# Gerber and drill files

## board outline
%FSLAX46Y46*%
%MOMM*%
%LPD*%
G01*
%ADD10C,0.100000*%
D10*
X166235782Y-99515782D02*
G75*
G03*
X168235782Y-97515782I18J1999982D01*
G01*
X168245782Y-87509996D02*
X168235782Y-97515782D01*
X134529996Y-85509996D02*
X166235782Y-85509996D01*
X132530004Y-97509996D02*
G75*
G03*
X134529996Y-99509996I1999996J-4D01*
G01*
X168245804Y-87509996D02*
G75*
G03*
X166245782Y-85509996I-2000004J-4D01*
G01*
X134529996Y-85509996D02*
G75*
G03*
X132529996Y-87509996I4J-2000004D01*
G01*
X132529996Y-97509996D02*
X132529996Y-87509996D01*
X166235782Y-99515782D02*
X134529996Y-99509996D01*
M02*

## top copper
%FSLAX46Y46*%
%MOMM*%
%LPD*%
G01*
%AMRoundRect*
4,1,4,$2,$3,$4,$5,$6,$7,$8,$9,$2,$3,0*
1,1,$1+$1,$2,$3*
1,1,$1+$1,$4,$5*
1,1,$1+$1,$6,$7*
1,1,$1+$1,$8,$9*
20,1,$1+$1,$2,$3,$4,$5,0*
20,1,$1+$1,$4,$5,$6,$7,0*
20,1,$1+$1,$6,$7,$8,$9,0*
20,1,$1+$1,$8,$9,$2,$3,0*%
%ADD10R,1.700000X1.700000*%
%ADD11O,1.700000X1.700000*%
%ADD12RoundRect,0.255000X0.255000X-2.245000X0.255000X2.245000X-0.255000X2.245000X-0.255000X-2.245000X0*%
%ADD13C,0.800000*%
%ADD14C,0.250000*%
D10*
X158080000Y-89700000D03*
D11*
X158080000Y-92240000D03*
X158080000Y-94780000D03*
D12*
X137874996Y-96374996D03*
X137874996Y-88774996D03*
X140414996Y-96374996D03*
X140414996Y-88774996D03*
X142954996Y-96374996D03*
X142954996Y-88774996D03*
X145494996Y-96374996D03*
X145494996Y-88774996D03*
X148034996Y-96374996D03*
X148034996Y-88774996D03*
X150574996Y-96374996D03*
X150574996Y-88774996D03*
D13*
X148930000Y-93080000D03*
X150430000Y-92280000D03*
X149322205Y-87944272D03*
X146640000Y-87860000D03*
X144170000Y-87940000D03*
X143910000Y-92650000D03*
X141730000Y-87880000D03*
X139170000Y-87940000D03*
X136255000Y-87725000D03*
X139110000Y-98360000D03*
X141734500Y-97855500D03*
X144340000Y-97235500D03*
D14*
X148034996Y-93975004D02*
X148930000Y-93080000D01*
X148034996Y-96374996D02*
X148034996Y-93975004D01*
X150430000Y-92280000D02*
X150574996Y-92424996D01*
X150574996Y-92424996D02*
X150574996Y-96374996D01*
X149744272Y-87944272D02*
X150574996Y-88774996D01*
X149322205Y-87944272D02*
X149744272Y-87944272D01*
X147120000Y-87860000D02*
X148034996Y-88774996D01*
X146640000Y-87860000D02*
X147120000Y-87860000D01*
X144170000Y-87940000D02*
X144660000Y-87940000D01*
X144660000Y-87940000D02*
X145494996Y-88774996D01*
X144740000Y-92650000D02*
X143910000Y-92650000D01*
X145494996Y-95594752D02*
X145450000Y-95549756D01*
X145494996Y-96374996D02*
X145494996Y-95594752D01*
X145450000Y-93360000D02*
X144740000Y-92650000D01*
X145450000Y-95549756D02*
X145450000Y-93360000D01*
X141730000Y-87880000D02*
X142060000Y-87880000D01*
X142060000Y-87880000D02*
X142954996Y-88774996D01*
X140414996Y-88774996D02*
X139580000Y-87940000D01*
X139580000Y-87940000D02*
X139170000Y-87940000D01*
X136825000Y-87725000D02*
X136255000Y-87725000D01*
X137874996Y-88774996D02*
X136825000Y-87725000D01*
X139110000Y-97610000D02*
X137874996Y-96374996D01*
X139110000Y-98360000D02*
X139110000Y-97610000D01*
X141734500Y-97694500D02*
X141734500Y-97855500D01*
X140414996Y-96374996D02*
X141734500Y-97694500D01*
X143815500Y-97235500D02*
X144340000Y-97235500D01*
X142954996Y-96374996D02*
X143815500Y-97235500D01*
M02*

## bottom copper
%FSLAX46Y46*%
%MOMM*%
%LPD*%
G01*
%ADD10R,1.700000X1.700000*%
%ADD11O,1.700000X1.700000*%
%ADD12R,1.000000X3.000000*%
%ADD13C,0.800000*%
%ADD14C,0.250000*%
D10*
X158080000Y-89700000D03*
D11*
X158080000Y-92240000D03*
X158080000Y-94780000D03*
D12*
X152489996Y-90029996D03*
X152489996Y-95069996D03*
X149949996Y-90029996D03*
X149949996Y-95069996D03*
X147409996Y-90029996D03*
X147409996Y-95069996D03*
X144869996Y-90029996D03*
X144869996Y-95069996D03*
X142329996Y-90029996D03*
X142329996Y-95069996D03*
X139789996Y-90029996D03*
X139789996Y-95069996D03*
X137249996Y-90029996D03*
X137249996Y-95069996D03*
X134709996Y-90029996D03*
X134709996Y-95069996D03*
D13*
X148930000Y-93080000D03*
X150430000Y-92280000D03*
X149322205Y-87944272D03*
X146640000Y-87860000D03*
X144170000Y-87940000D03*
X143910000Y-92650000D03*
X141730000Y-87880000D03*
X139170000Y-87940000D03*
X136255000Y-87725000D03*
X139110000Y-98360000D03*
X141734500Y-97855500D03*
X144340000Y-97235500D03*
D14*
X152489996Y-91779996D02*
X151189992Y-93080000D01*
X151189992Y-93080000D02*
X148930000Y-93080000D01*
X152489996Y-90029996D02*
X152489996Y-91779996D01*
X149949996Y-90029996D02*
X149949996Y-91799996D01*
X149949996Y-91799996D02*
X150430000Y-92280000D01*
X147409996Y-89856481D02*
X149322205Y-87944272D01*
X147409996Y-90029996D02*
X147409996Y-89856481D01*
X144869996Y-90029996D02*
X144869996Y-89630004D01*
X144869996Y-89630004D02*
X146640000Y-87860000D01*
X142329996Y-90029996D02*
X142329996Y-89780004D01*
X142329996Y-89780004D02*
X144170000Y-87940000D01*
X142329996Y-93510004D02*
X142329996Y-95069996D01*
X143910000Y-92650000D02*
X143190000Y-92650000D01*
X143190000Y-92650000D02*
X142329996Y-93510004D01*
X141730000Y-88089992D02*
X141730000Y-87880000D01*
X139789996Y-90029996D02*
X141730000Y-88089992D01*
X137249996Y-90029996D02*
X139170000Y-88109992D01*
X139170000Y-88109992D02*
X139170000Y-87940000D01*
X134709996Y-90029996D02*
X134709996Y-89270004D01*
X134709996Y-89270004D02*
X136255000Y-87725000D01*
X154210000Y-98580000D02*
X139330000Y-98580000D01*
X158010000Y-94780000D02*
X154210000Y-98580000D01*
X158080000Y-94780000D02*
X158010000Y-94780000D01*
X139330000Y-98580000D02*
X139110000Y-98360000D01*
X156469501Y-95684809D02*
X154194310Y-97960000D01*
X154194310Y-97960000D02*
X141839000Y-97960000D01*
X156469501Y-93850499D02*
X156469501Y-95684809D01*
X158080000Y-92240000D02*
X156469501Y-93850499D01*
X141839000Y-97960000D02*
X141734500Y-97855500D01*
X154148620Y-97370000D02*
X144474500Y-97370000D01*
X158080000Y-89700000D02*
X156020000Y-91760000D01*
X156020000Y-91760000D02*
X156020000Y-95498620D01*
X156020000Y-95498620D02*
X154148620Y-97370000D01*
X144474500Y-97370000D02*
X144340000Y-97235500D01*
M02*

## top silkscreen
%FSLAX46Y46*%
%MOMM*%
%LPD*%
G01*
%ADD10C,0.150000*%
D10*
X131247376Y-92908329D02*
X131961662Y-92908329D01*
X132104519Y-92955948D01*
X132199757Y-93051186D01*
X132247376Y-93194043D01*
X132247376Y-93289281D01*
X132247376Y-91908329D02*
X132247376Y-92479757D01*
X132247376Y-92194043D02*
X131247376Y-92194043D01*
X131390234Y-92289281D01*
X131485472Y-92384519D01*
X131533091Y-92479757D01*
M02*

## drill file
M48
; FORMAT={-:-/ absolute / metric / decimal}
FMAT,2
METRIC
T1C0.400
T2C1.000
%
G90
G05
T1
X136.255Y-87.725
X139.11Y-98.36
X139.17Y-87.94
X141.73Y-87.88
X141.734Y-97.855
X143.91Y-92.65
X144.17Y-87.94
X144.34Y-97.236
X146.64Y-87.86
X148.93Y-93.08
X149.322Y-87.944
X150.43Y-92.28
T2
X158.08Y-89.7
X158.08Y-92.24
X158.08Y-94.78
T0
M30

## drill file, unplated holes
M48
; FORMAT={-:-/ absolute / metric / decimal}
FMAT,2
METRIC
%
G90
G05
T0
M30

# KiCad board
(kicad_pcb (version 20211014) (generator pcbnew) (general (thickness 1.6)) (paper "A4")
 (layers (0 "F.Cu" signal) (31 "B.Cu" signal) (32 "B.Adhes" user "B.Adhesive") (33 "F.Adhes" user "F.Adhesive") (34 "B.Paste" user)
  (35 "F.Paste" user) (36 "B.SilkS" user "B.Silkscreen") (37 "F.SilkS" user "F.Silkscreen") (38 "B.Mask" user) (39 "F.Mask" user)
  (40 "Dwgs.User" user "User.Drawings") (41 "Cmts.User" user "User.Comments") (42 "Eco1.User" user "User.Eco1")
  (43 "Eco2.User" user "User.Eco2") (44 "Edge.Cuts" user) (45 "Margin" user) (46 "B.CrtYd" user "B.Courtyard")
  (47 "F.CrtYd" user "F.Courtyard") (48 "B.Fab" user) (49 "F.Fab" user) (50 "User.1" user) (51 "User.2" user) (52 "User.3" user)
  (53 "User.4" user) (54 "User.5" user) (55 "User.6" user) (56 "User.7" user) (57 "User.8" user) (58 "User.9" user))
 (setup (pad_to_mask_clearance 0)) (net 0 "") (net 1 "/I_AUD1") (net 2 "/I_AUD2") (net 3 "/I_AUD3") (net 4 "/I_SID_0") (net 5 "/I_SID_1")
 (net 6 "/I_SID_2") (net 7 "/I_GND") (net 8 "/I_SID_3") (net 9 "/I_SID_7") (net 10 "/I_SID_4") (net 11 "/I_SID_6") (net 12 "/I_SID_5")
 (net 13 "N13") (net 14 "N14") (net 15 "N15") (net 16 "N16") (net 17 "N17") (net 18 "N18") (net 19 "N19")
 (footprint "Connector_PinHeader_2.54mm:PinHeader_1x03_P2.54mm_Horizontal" (layer "F.Cu") (at 158.08 89.7)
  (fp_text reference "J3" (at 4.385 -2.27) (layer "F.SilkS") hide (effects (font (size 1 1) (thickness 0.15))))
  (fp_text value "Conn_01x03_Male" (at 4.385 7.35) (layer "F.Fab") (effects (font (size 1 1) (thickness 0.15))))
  (pad "1" thru_hole rect (at 0 0) (size 1.7 1.7) (drill 1) (layers *.Cu *.Mask) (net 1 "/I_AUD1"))
  (pad "2" thru_hole oval (at 0 2.54) (size 1.7 1.7) (drill 1) (layers *.Cu *.Mask) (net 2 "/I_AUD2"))
  (pad "3" thru_hole oval (at 0 5.08) (size 1.7 1.7) (drill 1) (layers *.Cu *.Mask) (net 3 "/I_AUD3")))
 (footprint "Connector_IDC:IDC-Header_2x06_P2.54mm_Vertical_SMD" (layer "F.Cu") (at 144.224996 92.574996 90)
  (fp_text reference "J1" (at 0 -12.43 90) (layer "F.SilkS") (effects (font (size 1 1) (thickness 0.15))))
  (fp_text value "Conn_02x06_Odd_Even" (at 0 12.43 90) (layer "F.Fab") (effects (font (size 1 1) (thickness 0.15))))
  (pad "1" smd roundrect (at -3.8 -6.35 90) (size 5 1.02) (layers "F.Cu" "F.Paste" "F.Mask") (roundrect_rratio 0.25) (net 3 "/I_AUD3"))
  (pad "2" smd roundrect (at 3.8 -6.35 90) (size 5 1.02) (layers "F.Cu" "F.Paste" "F.Mask") (roundrect_rratio 0.25) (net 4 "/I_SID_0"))
  (pad "3" smd roundrect (at -3.8 -3.81 90) (size 5 1.02) (layers "F.Cu" "F.Paste" "F.Mask") (roundrect_rratio 0.25) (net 2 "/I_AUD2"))
  (pad "4" smd roundrect (at 3.8 -3.81 90) (size 5 1.02) (layers "F.Cu" "F.Paste" "F.Mask") (roundrect_rratio 0.25) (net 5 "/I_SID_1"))
  (pad "5" smd roundrect (at -3.8 -1.27 90) (size 5 1.02) (layers "F.Cu" "F.Paste" "F.Mask") (roundrect_rratio 0.25) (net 1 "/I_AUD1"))
  (pad "6" smd roundrect (at 3.8 -1.27 90) (size 5 1.02) (layers "F.Cu" "F.Paste" "F.Mask") (roundrect_rratio 0.25) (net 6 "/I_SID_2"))
  (pad "7" smd roundrect (at -3.8 1.27 90) (size 5 1.02) (layers "F.Cu" "F.Paste" "F.Mask") (roundrect_rratio 0.25) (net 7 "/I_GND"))
  (pad "8" smd roundrect (at 3.8 1.27 90) (size 5 1.02) (layers "F.Cu" "F.Paste" "F.Mask") (roundrect_rratio 0.25) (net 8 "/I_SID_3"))
  (pad "9" smd roundrect (at -3.8 3.81 90) (size 5 1.02) (layers "F.Cu" "F.Paste" "F.Mask") (roundrect_rratio 0.25) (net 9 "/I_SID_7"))
  (pad "10" smd roundrect (at 3.8 3.81 90) (size 5 1.02) (layers "F.Cu" "F.Paste" "F.Mask") (roundrect_rratio 0.25) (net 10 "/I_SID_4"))
  (pad "11" smd roundrect (at -3.8 6.35 90) (size 5 1.02) (layers "F.Cu" "F.Paste" "F.Mask") (roundrect_rratio 0.25) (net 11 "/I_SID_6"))
  (pad "12" smd roundrect (at 3.8 6.35 90) (size 5 1.02) (layers "F.Cu" "F.Paste" "F.Mask") (roundrect_rratio 0.25) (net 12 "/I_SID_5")))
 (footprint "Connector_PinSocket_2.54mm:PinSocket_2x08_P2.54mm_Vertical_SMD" (layer "B.Cu") (at 143.599996 92.549996 90)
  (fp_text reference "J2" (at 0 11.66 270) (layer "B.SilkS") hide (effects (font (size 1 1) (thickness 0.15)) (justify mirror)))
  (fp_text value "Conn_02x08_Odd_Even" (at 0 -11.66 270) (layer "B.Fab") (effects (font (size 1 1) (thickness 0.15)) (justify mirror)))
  (pad "1" smd rect (at 2.52 8.89 90) (size 3 1) (layers "B.Cu" "B.Paste" "B.Mask") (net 9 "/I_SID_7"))
  (pad "2" smd rect (at -2.52 8.89 90) (size 3 1) (layers "B.Cu" "B.Paste" "B.Mask") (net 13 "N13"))
  (pad "3" smd rect (at 2.52 6.35 90) (size 3 1) (layers "B.Cu" "B.Paste" "B.Mask") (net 11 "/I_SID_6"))
  (pad "4" smd rect (at -2.52 6.35 90) (size 3 1) (layers "B.Cu" "B.Paste" "B.Mask") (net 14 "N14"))
  (pad "5" smd rect (at 2.52 3.81 90) (size 3 1) (layers "B.Cu" "B.Paste" "B.Mask") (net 12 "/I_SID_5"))
  (pad "6" smd rect (at -2.52 3.81 90) (size 3 1) (layers "B.Cu" "B.Paste" "B.Mask") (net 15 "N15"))
  (pad "7" smd rect (at 2.52 1.27 90) (size 3 1) (layers "B.Cu" "B.Paste" "B.Mask") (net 10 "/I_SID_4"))
  (pad "8" smd rect (at -2.52 1.27 90) (size 3 1) (layers "B.Cu" "B.Paste" "B.Mask") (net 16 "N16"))
  (pad "9" smd rect (at 2.52 -1.27 90) (size 3 1) (layers "B.Cu" "B.Paste" "B.Mask") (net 8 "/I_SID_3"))
  (pad "10" smd rect (at -2.52 -1.27 90) (size 3 1) (layers "B.Cu" "B.Paste" "B.Mask") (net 7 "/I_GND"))
  (pad "11" smd rect (at 2.52 -3.81 90) (size 3 1) (layers "B.Cu" "B.Paste" "B.Mask") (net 6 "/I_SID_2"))
  (pad "12" smd rect (at -2.52 -3.81 90) (size 3 1) (layers "B.Cu" "B.Paste" "B.Mask") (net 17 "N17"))
  (pad "13" smd rect (at 2.52 -6.35 90) (size 3 1) (layers "B.Cu" "B.Paste" "B.Mask") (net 5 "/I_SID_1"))
  (pad "14" smd rect (at -2.52 -6.35 90) (size 3 1) (layers "B.Cu" "B.Paste" "B.Mask") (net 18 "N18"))
  (pad "15" smd rect (at 2.52 -8.89 90) (size 3 1) (layers "B.Cu" "B.Paste" "B.Mask") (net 4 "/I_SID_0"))
  (pad "16" smd rect (at -2.52 -8.89 90) (size 3 1) (layers "B.Cu" "B.Paste" "B.Mask") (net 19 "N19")))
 (gr_arc (start 168.235782 97.515782) (mid 167.650001 98.930001) (end 166.235782 99.515782) (layer "Edge.Cuts") (width 0.1))
 (gr_line (start 168.245782 87.509996) (end 168.235782 97.515782) (layer "Edge.Cuts") (width 0.1))
 (gr_line (start 134.529996 85.509996) (end 166.235782 85.509996) (layer "Edge.Cuts") (width 0.1))
 (gr_arc (start 134.529996 99.509996) (mid 133.115786 98.924208) (end 132.529996 97.509996) (layer "Edge.Cuts") (width 0.1))
 (gr_arc (start 166.245782 85.509996) (mid 167.660009 86.095776) (end 168.245782 87.509996) (layer "Edge.Cuts") (width 0.1))
 (gr_arc (start 132.529996 87.509996) (mid 133.115784 86.095784) (end 134.529996 85.509996) (layer "Edge.Cuts") (width 0.1))
 (gr_line (start 132.529996 97.509996) (end 132.529996 87.509996) (layer "Edge.Cuts") (width 0.1))
 (gr_line (start 166.235782 99.515782) (end 134.529996 99.509996) (layer "Edge.Cuts") (width 0.1))
 (segment (start 148.034996 93.975004) (end 148.93 93.08) (width 0.25) (layer "F.Cu") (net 9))
 (segment (start 148.034996 96.374996) (end 148.034996 93.975004) (width 0.25) (layer "F.Cu") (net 9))
 (via (at 148.93 93.08) (size 0.8) (drill 0.4) (layers "F.Cu" "B.Cu") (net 9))
 (segment (start 152.489996 91.779996) (end 151.189992 93.08) (width 0.25) (layer "B.Cu") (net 9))
 (segment (start 151.189992 93.08) (end 148.93 93.08) (width 0.25) (layer "B.Cu") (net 9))
 (segment (start 152.489996 90.029996) (end 152.489996 91.779996) (width 0.25) (layer "B.Cu") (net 9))
 (segment (start 150.43 92.28) (end 150.574996 92.424996) (width 0.25) (layer "F.Cu") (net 11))
 (segment (start 150.574996 92.424996) (end 150.574996 96.374996) (width 0.25) (layer "F.Cu") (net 11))
 (via (at 150.43 92.28) (size 0.8) (drill 0.4) (layers "F.Cu" "B.Cu") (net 11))
 (segment (start 149.949996 90.029996) (end 149.949996 91.799996) (width 0.25) (layer "B.Cu") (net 11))
 (segment (start 149.949996 91.799996) (end 150.43 92.28) (width 0.25) (layer "B.Cu") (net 11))
 (segment (start 149.744272 87.944272) (end 150.574996 88.774996) (width 0.25) (layer "F.Cu") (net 12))
 (segment (start 149.322205 87.944272) (end 149.744272 87.944272) (width 0.25) (layer "F.Cu") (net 12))
 (via (at 149.322205 87.944272) (size 0.8) (drill 0.4) (layers "F.Cu" "B.Cu") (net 12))
 (segment (start 147.409996 89.856481) (end 149.322205 87.944272) (width 0.25) (layer "B.Cu") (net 12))
 (segment (start 147.409996 90.029996) (end 147.409996 89.856481) (width 0.25) (layer "B.Cu") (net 12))
 (segment (start 147.12 87.86) (end 148.034996 88.774996) (width 0.25) (layer "F.Cu") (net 10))
 (segment (start 146.64 87.86) (end 147.12 87.86) (width 0.25) (layer "F.Cu") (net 10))
 (via (at 146.64 87.86) (size 0.8) (drill 0.4) (layers "F.Cu" "B.Cu") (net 10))
 (segment (start 144.869996 90.029996) (end 144.869996 89.630004) (width 0.25) (layer "B.Cu") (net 10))
 (segment (start 144.869996 89.630004) (end 146.64 87.86) (width 0.25) (layer "B.Cu") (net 10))
 (segment (start 144.17 87.94) (end 144.66 87.94) (width 0.25) (layer "F.Cu") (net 8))
 (segment (start 144.66 87.94) (end 145.494996 88.774996) (width 0.25) (layer "F.Cu") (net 8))
 (via (at 144.17 87.94) (size 0.8) (drill 0.4) (layers "F.Cu" "B.Cu") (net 8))
 (segment (start 142.329996 90.029996) (end 142.329996 89.780004) (width 0.25) (layer "B.Cu") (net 8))
 (segment (start 142.329996 89.780004) (end 144.17 87.94) (width 0.25) (layer "B.Cu") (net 8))
 (segment (start 144.74 92.65) (end 143.91 92.65) (width 0.25) (layer "F.Cu") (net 7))
 (segment (start 145.494996 95.594752) (end 145.45 95.549756) (width 0.25) (layer "F.Cu") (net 7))
 (segment (start 145.494996 96.374996) (end 145.494996 95.594752) (width 0.25) (layer "F.Cu") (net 7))
 (segment (start 145.45 93.36) (end 144.74 92.65) (width 0.25) (layer "F.Cu") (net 7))
 (segment (start 145.45 95.549756) (end 145.45 93.36) (width 0.25) (layer "F.Cu") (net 7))
 (via (at 143.91 92.65) (size 0.8) (drill 0.4) (layers "F.Cu" "B.Cu") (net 7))
 (segment (start 142.329996 93.510004) (end 142.329996 95.069996) (width 0.25) (layer "B.Cu") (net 7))
 (segment (start 143.91 92.65) (end 143.19 92.65) (width 0.25) (layer "B.Cu") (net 7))
 (segment (start 143.19 92.65) (end 142.329996 93.510004) (width 0.25) (layer "B.Cu") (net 7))
 (segment (start 141.73 87.88) (end 142.06 87.88) (width 0.25) (layer "F.Cu") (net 6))
 (segment (start 142.06 87.88) (end 142.954996 88.774996) (width 0.25) (layer "F.Cu") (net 6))
 (via (at 141.73 87.88) (size 0.8) (drill 0.4) (layers "F.Cu" "B.Cu") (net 6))
 (segment (start 141.73 88.089992) (end 141.73 87.88) (width 0.25) (layer "B.Cu") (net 6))
 (segment (start 139.789996 90.029996) (end 141.73 88.089992) (width 0.25) (layer "B.Cu") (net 6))
 (segment (start 140.414996 88.774996) (end 139.58 87.94) (width 0.25) (layer "F.Cu") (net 5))
 (segment (start 139.58 87.94) (end 139.17 87.94) (width 0.25) (layer "F.Cu") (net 5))
 (via (at 139.17 87.94) (size 0.8) (drill 0.4) (layers "F.Cu" "B.Cu") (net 5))
 (segment (start 137.249996 90.029996) (end 139.17 88.109992) (width 0.25) (layer "B.Cu") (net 5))
 (segment (start 139.17 88.109992) (end 139.17 87.94) (width 0.25) (layer "B.Cu") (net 5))
 (segment (start 136.825 87.725) (end 136.255 87.725) (width 0.25) (layer "F.Cu") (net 4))
 (segment (start 137.874996 88.774996) (end 136.825 87.725) (width 0.25) (layer "F.Cu") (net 4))
 (via (at 136.255 87.725) (size 0.8) (drill 0.4) (layers "F.Cu" "B.Cu") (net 4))
 (segment (start 134.709996 90.029996) (end 134.709996 89.270004) (width 0.25) (layer "B.Cu") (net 4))
 (segment (start 134.709996 89.270004) (end 136.255 87.725) (width 0.25) (layer "B.Cu") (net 4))
 (segment (start 139.11 97.61) (end 137.874996 96.374996) (width 0.25) (layer "F.Cu") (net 3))
 (segment (start 139.11 98.36) (end 139.11 97.61) (width 0.25) (layer "F.Cu") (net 3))
 (via (at 139.11 98.36) (size 0.8) (drill 0.4) (layers "F.Cu" "B.Cu") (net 3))
 (segment (start 154.21 98.58) (end 139.33 98.58) (width 0.25) (layer "B.Cu") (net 3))
 (segment (start 158.01 94.78) (end 154.21 98.58) (width 0.25) (layer "B.Cu") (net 3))
 (segment (start 158.08 94.78) (end 158.01 94.78) (width 0.25) (layer "B.Cu") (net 3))
 (segment (start 139.33 98.58) (end 139.11 98.36) (width 0.25) (layer "B.Cu") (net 3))
 (segment (start 141.7345 97.6945) (end 141.7345 97.8555) (width 0.25) (layer "F.Cu") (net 2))
 (segment (start 140.414996 96.374996) (end 141.7345 97.6945) (width 0.25) (layer "F.Cu") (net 2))
 (via (at 141.7345 97.8555) (size 0.8) (drill 0.4) (layers "F.Cu" "B.Cu") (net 2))
 (segment (start 156.469501 95.684809) (end 154.19431 97.96) (width 0.25) (layer "B.Cu") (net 2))
 (segment (start 154.19431 97.96) (end 141.839 97.96) (width 0.25) (layer "B.Cu") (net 2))
 (segment (start 156.469501 93.850499) (end 156.469501 95.684809) (width 0.25) (layer "B.Cu") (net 2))
 (segment (start 158.08 92.24) (end 156.469501 93.850499) (width 0.25) (layer "B.Cu") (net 2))
 (segment (start 141.839 97.96) (end 141.7345 97.8555) (width 0.25) (layer "B.Cu") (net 2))
 (segment (start 143.8155 97.2355) (end 144.34 97.2355) (width 0.25) (layer "F.Cu") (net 1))
 (segment (start 142.954996 96.374996) (end 143.8155 97.2355) (width 0.25) (layer "F.Cu") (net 1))
 (via (at 144.34 97.2355) (size 0.8) (drill 0.4) (layers "F.Cu" "B.Cu") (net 1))
 (segment (start 154.14862 97.37) (end 144.4745 97.37) (width 0.25) (layer "B.Cu") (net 1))
 (segment (start 158.08 89.7) (end 156.02 91.76) (width 0.25) (layer "B.Cu") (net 1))
 (segment (start 156.02 91.76) (end 156.02 95.49862) (width 0.25) (layer "B.Cu") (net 1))
 (segment (start 156.02 95.49862) (end 154.14862 97.37) (width 0.25) (layer "B.Cu") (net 1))
 (segment (start 144.4745 97.37) (end 144.34 97.2355) (width 0.25) (layer "B.Cu") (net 1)))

